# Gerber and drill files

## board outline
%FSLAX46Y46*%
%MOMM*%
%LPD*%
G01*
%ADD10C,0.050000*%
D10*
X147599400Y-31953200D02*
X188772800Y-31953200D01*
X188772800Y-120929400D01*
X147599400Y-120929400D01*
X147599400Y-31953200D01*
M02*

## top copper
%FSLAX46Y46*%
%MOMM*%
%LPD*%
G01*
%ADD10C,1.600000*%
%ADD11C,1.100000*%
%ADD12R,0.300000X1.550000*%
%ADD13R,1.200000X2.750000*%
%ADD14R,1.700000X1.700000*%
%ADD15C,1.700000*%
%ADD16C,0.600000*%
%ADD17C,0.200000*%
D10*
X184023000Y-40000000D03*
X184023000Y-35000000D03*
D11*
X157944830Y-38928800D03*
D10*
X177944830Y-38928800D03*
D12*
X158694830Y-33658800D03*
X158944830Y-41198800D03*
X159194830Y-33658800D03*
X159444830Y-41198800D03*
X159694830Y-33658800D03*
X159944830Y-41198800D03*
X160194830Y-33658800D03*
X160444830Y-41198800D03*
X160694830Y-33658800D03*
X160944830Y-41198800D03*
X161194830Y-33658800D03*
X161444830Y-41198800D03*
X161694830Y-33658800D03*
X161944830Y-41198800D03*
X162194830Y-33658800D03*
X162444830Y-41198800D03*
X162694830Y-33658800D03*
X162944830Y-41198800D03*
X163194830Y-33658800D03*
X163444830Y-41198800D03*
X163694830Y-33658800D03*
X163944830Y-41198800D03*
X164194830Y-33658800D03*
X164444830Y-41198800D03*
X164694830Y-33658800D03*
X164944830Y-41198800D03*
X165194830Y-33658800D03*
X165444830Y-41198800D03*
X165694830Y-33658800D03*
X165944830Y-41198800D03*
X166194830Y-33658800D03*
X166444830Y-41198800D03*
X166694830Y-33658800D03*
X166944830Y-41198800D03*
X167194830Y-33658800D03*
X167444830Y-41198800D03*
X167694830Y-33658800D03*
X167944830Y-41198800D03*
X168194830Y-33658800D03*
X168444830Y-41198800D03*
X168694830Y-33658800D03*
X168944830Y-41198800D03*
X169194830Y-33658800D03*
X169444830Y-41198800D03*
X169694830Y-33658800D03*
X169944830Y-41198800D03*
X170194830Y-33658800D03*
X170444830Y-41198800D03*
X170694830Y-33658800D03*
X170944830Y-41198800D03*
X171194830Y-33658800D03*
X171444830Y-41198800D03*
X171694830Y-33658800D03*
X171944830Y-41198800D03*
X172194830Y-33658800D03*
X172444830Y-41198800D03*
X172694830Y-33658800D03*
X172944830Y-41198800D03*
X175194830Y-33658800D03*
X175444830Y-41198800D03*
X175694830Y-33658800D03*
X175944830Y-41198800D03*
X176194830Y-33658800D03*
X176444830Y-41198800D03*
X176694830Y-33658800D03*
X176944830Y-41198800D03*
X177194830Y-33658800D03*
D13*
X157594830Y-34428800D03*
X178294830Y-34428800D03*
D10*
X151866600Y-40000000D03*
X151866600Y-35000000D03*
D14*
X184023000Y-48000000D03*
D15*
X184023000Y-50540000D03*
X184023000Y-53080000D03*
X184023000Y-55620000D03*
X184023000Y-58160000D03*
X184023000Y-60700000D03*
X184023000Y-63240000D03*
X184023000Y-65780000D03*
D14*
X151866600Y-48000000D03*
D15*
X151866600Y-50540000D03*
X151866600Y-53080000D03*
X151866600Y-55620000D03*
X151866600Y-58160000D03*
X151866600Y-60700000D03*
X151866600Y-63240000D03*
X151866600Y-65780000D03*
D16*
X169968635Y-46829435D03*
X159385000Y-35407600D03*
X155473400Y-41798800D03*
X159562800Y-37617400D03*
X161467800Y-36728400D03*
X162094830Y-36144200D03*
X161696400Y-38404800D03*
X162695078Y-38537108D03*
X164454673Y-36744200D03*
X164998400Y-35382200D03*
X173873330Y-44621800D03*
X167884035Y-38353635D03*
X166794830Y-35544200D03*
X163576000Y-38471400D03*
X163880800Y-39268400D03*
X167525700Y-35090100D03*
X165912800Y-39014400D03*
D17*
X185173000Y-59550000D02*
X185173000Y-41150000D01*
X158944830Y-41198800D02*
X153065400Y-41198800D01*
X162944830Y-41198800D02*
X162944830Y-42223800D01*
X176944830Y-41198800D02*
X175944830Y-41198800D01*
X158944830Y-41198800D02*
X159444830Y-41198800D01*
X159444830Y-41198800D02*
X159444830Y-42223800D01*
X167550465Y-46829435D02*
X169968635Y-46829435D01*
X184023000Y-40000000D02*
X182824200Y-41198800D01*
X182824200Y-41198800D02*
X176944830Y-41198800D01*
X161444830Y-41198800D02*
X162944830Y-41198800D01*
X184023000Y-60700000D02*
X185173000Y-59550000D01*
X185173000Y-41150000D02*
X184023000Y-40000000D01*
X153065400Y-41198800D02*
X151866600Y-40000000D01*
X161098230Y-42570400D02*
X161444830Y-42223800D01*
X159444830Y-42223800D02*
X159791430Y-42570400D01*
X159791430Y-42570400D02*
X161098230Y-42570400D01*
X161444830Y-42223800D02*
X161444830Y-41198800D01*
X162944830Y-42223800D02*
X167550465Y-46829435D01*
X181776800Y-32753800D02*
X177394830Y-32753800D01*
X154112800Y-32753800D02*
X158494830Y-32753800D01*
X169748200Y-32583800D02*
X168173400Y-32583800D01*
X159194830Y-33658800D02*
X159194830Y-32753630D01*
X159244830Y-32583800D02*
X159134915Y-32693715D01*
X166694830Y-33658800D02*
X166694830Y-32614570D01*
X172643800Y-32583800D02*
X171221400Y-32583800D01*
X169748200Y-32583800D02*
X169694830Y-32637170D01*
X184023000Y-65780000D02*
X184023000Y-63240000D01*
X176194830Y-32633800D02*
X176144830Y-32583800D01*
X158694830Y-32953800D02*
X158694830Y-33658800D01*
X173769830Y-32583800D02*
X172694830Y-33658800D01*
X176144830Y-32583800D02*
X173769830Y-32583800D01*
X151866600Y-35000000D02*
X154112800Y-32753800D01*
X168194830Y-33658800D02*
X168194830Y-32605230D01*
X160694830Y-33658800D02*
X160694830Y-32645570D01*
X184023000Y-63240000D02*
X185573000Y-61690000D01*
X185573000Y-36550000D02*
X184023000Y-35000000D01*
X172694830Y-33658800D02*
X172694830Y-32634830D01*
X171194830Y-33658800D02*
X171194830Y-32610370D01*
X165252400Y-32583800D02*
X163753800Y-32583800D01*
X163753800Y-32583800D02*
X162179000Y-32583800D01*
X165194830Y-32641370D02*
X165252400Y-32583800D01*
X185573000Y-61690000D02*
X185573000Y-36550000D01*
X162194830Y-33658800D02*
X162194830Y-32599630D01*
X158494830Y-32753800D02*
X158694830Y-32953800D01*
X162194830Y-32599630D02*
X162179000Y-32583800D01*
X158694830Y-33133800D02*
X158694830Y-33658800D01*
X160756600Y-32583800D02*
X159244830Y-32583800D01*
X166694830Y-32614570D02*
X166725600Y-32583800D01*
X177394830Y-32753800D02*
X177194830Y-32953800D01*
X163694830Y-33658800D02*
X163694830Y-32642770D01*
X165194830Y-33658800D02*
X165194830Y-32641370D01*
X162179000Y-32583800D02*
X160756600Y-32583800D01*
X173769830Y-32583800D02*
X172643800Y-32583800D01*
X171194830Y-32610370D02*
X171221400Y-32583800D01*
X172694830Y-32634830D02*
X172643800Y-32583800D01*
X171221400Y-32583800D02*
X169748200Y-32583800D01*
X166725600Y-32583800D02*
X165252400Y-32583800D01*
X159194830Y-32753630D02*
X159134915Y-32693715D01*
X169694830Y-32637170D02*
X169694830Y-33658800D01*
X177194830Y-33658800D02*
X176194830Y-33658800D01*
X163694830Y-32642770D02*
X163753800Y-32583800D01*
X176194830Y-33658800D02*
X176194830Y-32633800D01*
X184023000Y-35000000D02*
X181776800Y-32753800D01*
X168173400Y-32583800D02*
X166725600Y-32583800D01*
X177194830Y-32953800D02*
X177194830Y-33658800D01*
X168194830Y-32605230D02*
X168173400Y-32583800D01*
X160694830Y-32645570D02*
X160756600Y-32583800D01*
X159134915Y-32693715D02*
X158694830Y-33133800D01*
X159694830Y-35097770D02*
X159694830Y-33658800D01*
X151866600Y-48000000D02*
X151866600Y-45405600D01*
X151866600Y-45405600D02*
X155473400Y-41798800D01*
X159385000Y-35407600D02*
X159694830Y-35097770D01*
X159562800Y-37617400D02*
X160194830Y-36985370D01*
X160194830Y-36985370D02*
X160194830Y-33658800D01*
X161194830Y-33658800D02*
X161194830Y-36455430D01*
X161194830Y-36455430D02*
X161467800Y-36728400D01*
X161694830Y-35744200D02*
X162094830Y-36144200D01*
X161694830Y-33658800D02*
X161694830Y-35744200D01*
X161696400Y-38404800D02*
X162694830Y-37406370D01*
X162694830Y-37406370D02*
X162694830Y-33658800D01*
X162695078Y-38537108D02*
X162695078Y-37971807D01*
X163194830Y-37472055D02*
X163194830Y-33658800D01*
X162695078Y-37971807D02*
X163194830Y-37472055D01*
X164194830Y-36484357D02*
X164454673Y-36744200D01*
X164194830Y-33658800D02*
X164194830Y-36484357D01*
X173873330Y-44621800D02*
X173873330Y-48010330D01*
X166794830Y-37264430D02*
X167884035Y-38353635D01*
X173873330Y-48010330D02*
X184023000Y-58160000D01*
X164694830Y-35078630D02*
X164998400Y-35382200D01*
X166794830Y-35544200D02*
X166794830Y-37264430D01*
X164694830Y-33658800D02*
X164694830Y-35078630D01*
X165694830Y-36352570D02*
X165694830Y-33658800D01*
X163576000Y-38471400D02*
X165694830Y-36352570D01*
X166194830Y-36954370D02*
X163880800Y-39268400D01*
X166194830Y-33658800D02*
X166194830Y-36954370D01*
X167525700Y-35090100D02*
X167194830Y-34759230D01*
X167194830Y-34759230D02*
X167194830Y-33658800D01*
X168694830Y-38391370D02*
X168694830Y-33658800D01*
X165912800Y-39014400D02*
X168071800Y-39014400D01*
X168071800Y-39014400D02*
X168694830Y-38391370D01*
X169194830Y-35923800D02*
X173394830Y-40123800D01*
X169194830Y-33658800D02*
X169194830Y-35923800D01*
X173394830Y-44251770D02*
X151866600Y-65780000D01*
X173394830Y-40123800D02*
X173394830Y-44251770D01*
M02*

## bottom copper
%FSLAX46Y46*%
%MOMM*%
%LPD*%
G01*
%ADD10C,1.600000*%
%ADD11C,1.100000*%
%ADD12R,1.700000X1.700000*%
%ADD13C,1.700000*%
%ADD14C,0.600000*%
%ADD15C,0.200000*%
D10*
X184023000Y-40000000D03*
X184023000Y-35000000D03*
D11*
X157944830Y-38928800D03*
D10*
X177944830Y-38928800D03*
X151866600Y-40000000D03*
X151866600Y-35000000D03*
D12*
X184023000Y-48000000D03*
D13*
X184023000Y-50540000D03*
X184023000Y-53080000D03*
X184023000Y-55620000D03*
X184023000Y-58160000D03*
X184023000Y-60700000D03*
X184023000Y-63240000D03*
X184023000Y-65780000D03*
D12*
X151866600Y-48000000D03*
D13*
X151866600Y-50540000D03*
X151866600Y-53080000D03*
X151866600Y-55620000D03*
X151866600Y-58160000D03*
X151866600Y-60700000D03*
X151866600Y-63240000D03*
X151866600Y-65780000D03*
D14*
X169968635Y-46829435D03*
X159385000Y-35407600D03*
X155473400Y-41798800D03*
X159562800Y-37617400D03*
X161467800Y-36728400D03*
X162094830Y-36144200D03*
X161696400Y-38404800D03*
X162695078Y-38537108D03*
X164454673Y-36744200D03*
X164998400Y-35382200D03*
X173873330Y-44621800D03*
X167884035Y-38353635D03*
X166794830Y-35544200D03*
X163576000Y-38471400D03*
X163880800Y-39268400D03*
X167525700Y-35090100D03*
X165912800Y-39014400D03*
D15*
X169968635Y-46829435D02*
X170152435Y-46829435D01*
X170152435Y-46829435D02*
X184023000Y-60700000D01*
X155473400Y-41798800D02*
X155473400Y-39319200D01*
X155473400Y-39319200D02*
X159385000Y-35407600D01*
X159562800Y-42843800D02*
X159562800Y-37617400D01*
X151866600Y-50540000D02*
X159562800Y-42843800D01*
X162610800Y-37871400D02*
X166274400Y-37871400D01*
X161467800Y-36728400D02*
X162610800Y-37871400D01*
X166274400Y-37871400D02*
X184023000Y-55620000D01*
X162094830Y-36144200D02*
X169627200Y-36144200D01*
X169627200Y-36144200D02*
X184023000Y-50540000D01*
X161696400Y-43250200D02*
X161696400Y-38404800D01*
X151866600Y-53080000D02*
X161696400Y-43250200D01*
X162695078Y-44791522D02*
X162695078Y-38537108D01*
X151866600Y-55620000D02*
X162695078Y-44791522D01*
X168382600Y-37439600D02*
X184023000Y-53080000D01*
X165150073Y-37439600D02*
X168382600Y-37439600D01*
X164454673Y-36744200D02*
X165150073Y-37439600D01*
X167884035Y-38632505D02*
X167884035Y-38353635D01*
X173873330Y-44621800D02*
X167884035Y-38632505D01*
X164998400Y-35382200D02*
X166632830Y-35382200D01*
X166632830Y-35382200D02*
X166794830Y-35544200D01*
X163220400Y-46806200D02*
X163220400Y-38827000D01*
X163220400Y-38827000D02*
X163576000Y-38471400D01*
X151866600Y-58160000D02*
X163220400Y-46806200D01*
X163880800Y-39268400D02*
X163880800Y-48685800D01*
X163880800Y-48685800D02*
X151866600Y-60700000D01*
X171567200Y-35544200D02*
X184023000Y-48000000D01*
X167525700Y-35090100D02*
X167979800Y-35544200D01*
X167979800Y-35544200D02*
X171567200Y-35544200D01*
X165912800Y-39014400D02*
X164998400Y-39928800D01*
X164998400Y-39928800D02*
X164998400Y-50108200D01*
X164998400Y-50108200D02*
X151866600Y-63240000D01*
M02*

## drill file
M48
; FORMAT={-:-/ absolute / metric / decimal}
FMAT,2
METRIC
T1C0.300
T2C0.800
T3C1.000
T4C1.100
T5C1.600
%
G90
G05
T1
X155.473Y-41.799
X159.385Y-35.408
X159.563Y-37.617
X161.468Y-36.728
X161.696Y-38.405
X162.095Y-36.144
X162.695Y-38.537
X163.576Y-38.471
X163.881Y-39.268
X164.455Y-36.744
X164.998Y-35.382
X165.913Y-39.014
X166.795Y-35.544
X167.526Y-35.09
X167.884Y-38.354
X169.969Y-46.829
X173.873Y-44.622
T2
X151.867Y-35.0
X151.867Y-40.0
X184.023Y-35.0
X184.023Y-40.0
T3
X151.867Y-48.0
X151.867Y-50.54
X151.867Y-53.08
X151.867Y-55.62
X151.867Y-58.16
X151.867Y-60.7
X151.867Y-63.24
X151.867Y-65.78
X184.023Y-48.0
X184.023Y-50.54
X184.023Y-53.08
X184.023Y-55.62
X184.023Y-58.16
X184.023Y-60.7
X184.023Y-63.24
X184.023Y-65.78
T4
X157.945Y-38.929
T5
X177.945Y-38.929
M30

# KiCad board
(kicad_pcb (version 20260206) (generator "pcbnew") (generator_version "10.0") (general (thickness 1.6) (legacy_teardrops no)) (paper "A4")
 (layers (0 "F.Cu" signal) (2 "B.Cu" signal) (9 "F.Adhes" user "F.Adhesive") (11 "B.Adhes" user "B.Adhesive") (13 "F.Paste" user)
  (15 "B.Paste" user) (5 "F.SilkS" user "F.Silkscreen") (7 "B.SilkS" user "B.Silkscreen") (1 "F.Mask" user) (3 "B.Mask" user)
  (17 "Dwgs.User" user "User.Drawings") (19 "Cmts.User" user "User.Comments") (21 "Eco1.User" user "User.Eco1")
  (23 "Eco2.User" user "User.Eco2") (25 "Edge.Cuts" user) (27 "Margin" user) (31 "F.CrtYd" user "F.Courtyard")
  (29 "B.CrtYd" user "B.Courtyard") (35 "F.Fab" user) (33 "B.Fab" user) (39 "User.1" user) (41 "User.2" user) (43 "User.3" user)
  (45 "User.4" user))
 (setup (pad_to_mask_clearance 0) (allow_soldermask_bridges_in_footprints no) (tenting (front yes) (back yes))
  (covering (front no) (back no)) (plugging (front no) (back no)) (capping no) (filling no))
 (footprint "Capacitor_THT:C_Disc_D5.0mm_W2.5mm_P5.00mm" (layer "F.Cu") (at 184.023 40 90)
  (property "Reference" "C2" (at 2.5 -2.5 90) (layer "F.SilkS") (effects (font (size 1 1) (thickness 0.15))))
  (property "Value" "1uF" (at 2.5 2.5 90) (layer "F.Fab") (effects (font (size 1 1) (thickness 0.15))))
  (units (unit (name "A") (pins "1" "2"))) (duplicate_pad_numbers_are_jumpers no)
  (pad "1" thru_hole circle (at 0 0 90) (size 1.6 1.6) (drill 0.8) (layers "*.Cu" "*.Mask") (remove_unused_layers no) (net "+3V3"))
  (pad "2" thru_hole circle (at 5 0 90) (size 1.6 1.6) (drill 0.8) (layers "*.Cu" "*.Mask") (remove_unused_layers no) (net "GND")))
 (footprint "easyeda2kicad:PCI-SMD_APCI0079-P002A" (layer "F.Cu") (at 167.94483 37.4288)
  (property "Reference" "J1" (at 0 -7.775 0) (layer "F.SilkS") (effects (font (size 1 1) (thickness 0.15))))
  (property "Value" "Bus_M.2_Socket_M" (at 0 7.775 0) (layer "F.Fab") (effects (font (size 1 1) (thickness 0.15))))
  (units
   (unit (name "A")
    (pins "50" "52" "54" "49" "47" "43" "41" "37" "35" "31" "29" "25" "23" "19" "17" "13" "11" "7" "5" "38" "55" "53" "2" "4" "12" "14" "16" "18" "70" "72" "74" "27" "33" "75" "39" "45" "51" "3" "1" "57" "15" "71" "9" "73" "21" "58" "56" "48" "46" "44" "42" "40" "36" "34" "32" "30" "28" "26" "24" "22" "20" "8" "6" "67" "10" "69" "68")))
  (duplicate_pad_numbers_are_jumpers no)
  (pad "" thru_hole circle (at -10 1.5) (size 1.1 1.1) (drill 1.1) (layers "*.Cu" "*.Mask") (remove_unused_layers no))
  (pad "" thru_hole circle (at 10 1.5) (size 1.6 1.6) (drill 1.6) (layers "*.Cu" "*.Mask") (remove_unused_layers no))
  (pad "1" smd rect (at -9.25 -3.77) (size 0.3 1.55) (layers "F.Cu" "F.Mask" "F.Paste") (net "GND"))
  (pad "2" smd rect (at -9 3.77) (size 0.3 1.55) (layers "F.Cu" "F.Mask" "F.Paste") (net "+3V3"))
  (pad "3" smd rect (at -8.75 -3.77) (size 0.3 1.55) (layers "F.Cu" "F.Mask" "F.Paste") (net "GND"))
  (pad "4" smd rect (at -8.5 3.77) (size 0.3 1.55) (layers "F.Cu" "F.Mask" "F.Paste") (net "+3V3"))
  (pad "5" smd rect (at -8.25 -3.77) (size 0.3 1.55) (layers "F.Cu" "F.Mask" "F.Paste") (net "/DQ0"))
  (pad "6" smd rect (at -8 3.77) (size 0.3 1.55) (layers "F.Cu" "F.Mask" "F.Paste") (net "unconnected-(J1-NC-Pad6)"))
  (pad "7" smd rect (at -7.75 -3.77) (size 0.3 1.55) (layers "F.Cu" "F.Mask" "F.Paste") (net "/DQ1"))
  (pad "8" smd rect (at -7.5 3.77) (size 0.3 1.55) (layers "F.Cu" "F.Mask" "F.Paste") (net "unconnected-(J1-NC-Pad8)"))
  (pad "9" smd rect (at -7.25 -3.77) (size 0.3 1.55) (layers "F.Cu" "F.Mask" "F.Paste") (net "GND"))
  (pad "10" smd rect (at -7 3.77) (size 0.3 1.55) (layers "F.Cu" "F.Mask" "F.Paste")
   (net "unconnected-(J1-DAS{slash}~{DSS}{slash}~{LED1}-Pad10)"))
  (pad "11" smd rect (at -6.75 -3.77) (size 0.3 1.55) (layers "F.Cu" "F.Mask" "F.Paste") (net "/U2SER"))
  (pad "12" smd rect (at -6.5 3.77) (size 0.3 1.55) (layers "F.Cu" "F.Mask" "F.Paste") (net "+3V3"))
  (pad "13" smd rect (at -6.25 -3.77) (size 0.3 1.55) (layers "F.Cu" "F.Mask" "F.Paste") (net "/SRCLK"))
  (pad "14" smd rect (at -6 3.77) (size 0.3 1.55) (layers "F.Cu" "F.Mask" "F.Paste") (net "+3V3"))
  (pad "15" smd rect (at -5.75 -3.77) (size 0.3 1.55) (layers "F.Cu" "F.Mask" "F.Paste") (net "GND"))
  (pad "16" smd rect (at -5.5 3.77) (size 0.3 1.55) (layers "F.Cu" "F.Mask" "F.Paste") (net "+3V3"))
  (pad "17" smd rect (at -5.25 -3.77) (size 0.3 1.55) (layers "F.Cu" "F.Mask" "F.Paste") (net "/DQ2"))
  (pad "18" smd rect (at -5 3.77) (size 0.3 1.55) (layers "F.Cu" "F.Mask" "F.Paste") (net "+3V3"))
  (pad "19" smd rect (at -4.75 -3.77) (size 0.3 1.55) (layers "F.Cu" "F.Mask" "F.Paste") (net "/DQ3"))
  (pad "20" smd rect (at -4.5 3.77) (size 0.3 1.55) (layers "F.Cu" "F.Mask" "F.Paste") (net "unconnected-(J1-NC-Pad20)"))
  (pad "21" smd rect (at -4.25 -3.77) (size 0.3 1.55) (layers "F.Cu" "F.Mask" "F.Paste") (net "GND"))
  (pad "22" smd rect (at -4 3.77) (size 0.3 1.55) (layers "F.Cu" "F.Mask" "F.Paste") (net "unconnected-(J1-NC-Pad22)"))
  (pad "23" smd rect (at -3.75 -3.77) (size 0.3 1.55) (layers "F.Cu" "F.Mask" "F.Paste") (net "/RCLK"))
  (pad "24" smd rect (at -3.5 3.77) (size 0.3 1.55) (layers "F.Cu" "F.Mask" "F.Paste") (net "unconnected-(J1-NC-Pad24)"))
  (pad "25" smd rect (at -3.25 -3.77) (size 0.3 1.55) (layers "F.Cu" "F.Mask" "F.Paste") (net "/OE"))
  (pad "26" smd rect (at -3 3.77) (size 0.3 1.55) (layers "F.Cu" "F.Mask" "F.Paste") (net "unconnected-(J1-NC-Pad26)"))
  (pad "27" smd rect (at -2.75 -3.77) (size 0.3 1.55) (layers "F.Cu" "F.Mask" "F.Paste") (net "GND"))
  (pad "28" smd rect (at -2.5 3.77) (size 0.3 1.55) (layers "F.Cu" "F.Mask" "F.Paste") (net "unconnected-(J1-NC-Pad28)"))
  (pad "29" smd rect (at -2.25 -3.77) (size 0.3 1.55) (layers "F.Cu" "F.Mask" "F.Paste") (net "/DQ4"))
  (pad "30" smd rect (at -2 3.77) (size 0.3 1.55) (layers "F.Cu" "F.Mask" "F.Paste") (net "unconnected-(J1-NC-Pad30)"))
  (pad "31" smd rect (at -1.75 -3.77) (size 0.3 1.55) (layers "F.Cu" "F.Mask" "F.Paste") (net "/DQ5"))
  (pad "32" smd rect (at -1.5 3.77) (size 0.3 1.55) (layers "F.Cu" "F.Mask" "F.Paste") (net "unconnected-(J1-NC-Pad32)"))
  (pad "33" smd rect (at -1.25 -3.77) (size 0.3 1.55) (layers "F.Cu" "F.Mask" "F.Paste") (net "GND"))
  (pad "34" smd rect (at -1 3.77) (size 0.3 1.55) (layers "F.Cu" "F.Mask" "F.Paste") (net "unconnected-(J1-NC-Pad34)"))
  (pad "35" smd rect (at -0.75 -3.77) (size 0.3 1.55) (layers "F.Cu" "F.Mask" "F.Paste") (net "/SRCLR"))
  (pad "36" smd rect (at -0.5 3.77) (size 0.3 1.55) (layers "F.Cu" "F.Mask" "F.Paste") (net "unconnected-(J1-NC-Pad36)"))
  (pad "37" smd rect (at -0.25 -3.77) (size 0.3 1.55) (layers "F.Cu" "F.Mask" "F.Paste") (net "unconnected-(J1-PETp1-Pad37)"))
  (pad "38" smd rect (at 0 3.77) (size 0.3 1.55) (layers "F.Cu" "F.Mask" "F.Paste") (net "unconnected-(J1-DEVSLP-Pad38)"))
  (pad "39" smd rect (at 0.25 -3.77) (size 0.3 1.55) (layers "F.Cu" "F.Mask" "F.Paste") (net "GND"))
  (pad "40" smd rect (at 0.5 3.77) (size 0.3 1.55) (layers "F.Cu" "F.Mask" "F.Paste") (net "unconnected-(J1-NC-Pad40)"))
  (pad "41" smd rect (at 0.75 -3.77) (size 0.3 1.55) (layers "F.Cu" "F.Mask" "F.Paste") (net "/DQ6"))
  (pad "42" smd rect (at 1 3.77) (size 0.3 1.55) (layers "F.Cu" "F.Mask" "F.Paste") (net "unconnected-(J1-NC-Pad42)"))
  (pad "43" smd rect (at 1.25 -3.77) (size 0.3 1.55) (layers "F.Cu" "F.Mask" "F.Paste") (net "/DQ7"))
  (pad "44" smd rect (at 1.5 3.77) (size 0.3 1.55) (layers "F.Cu" "F.Mask" "F.Paste") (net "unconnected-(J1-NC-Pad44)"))
  (pad "45" smd rect (at 1.75 -3.77) (size 0.3 1.55) (layers "F.Cu" "F.Mask" "F.Paste") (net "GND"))
  (pad "46" smd rect (at 2 3.77) (size 0.3 1.55) (layers "F.Cu" "F.Mask" "F.Paste") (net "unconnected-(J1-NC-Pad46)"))
  (pad "47" smd rect (at 2.25 -3.77) (size 0.3 1.55) (layers "F.Cu" "F.Mask" "F.Paste") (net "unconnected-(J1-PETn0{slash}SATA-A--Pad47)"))
  (pad "48" smd rect (at 2.5 3.77) (size 0.3 1.55) (layers "F.Cu" "F.Mask" "F.Paste") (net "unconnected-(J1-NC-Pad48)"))
  (pad "49" smd rect (at 2.75 -3.77) (size 0.3 1.55) (layers "F.Cu" "F.Mask" "F.Paste") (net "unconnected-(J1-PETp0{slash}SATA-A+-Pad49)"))
  (pad "50" smd rect (at 3 3.77) (size 0.3 1.55) (layers "F.Cu" "F.Mask" "F.Paste") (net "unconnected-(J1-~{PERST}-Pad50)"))
  (pad "51" smd rect (at 3.25 -3.77) (size 0.3 1.55) (layers "F.Cu" "F.Mask" "F.Paste") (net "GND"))
  (pad "52" smd rect (at 3.5 3.77) (size 0.3 1.55) (layers "F.Cu" "F.Mask" "F.Paste") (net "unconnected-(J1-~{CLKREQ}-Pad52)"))
  (pad "53" smd rect (at 3.75 -3.77) (size 0.3 1.55) (layers "F.Cu" "F.Mask" "F.Paste") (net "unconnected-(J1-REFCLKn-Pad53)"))
  (pad "54" smd rect (at 4 3.77) (size 0.3 1.55) (layers "F.Cu" "F.Mask" "F.Paste") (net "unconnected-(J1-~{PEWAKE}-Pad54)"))
  (pad "55" smd rect (at 4.25 -3.77) (size 0.3 1.55) (layers "F.Cu" "F.Mask" "F.Paste") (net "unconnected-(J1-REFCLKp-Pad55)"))
  (pad "56" smd rect (at 4.5 3.77) (size 0.3 1.55) (layers "F.Cu" "F.Mask" "F.Paste") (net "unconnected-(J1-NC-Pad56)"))
  (pad "57" smd rect (at 4.75 -3.77) (size 0.3 1.55) (layers "F.Cu" "F.Mask" "F.Paste") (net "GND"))
  (pad "58" smd rect (at 5 3.77) (size 0.3 1.55) (layers "F.Cu" "F.Mask" "F.Paste") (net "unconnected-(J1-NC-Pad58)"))
  (pad "67" smd rect (at 7.25 -3.77) (size 0.3 1.55) (layers "F.Cu" "F.Mask" "F.Paste") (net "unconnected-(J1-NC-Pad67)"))
  (pad "68" smd rect (at 7.5 3.77) (size 0.3 1.55) (layers "F.Cu" "F.Mask" "F.Paste") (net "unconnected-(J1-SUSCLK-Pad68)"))
  (pad "69" smd rect (at 7.75 -3.77) (size 0.3 1.55) (layers "F.Cu" "F.Mask" "F.Paste") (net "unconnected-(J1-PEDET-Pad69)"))
  (pad "70" smd rect (at 8 3.77) (size 0.3 1.55) (layers "F.Cu" "F.Mask" "F.Paste") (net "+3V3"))
  (pad "71" smd rect (at 8.25 -3.77) (size 0.3 1.55) (layers "F.Cu" "F.Mask" "F.Paste") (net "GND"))
  (pad "72" smd rect (at 8.5 3.77) (size 0.3 1.55) (layers "F.Cu" "F.Mask" "F.Paste") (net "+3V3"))
  (pad "73" smd rect (at 8.75 -3.77) (size 0.3 1.55) (layers "F.Cu" "F.Mask" "F.Paste") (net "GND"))
  (pad "74" smd rect (at 9 3.77) (size 0.3 1.55) (layers "F.Cu" "F.Mask" "F.Paste") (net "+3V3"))
  (pad "75" smd rect (at 9.25 -3.77) (size 0.3 1.55) (layers "F.Cu" "F.Mask" "F.Paste") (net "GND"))
  (pad "76" smd rect (at -10.35 -3) (size 1.2 2.75) (layers "F.Cu" "F.Mask" "F.Paste"))
  (pad "76" smd rect (at 10.35 -3) (size 1.2 2.75) (layers "F.Cu" "F.Mask" "F.Paste")))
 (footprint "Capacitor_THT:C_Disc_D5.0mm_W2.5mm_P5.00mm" (layer "F.Cu") (at 151.8666 40 90)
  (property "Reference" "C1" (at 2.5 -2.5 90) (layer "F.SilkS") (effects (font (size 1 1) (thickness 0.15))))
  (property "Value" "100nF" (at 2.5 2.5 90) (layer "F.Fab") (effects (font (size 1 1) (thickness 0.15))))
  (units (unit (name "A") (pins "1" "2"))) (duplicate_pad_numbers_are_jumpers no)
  (pad "1" thru_hole circle (at 0 0 90) (size 1.6 1.6) (drill 0.8) (layers "*.Cu" "*.Mask") (remove_unused_layers no) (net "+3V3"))
  (pad "2" thru_hole circle (at 5 0 90) (size 1.6 1.6) (drill 0.8) (layers "*.Cu" "*.Mask") (remove_unused_layers no) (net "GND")))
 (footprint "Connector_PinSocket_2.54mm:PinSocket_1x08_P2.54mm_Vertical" (layer "F.Cu") (at 184.023 48)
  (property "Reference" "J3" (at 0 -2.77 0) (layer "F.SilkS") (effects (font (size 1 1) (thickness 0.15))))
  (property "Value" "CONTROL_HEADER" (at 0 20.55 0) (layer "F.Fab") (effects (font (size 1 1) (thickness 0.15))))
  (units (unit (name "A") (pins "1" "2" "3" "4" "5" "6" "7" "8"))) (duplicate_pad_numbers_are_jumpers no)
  (pad "1" thru_hole rect (at 0 0) (size 1.7 1.7) (drill 1) (layers "*.Cu" "*.Mask") (remove_unused_layers no) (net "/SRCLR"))
  (pad "2" thru_hole circle (at 0 2.54) (size 1.7 1.7) (drill 1) (layers "*.Cu" "*.Mask") (remove_unused_layers no) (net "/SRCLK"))
  (pad "3" thru_hole circle (at 0 5.08) (size 1.7 1.7) (drill 1) (layers "*.Cu" "*.Mask") (remove_unused_layers no) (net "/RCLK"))
  (pad "4" thru_hole circle (at 0 7.62) (size 1.7 1.7) (drill 1) (layers "*.Cu" "*.Mask") (remove_unused_layers no) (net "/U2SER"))
  (pad "5" thru_hole circle (at 0 10.16) (size 1.7 1.7) (drill 1) (layers "*.Cu" "*.Mask") (remove_unused_layers no) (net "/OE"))
  (pad "6" thru_hole circle (at 0 12.7) (size 1.7 1.7) (drill 1) (layers "*.Cu" "*.Mask") (remove_unused_layers no) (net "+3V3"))
  (pad "7" thru_hole circle (at 0 15.24) (size 1.7 1.7) (drill 1) (layers "*.Cu" "*.Mask") (remove_unused_layers no) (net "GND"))
  (pad "8" thru_hole circle (at 0 17.78) (size 1.7 1.7) (drill 1) (layers "*.Cu" "*.Mask") (remove_unused_layers no) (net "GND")))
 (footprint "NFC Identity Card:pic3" (layer "F.Cu") (at 168.148 111.0488)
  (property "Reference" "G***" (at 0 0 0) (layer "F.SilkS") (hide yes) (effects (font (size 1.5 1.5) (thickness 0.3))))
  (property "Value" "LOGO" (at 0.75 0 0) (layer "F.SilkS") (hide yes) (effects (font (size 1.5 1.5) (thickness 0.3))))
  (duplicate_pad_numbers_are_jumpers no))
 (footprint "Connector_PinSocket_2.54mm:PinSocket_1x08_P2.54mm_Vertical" (layer "F.Cu") (at 151.8666 48)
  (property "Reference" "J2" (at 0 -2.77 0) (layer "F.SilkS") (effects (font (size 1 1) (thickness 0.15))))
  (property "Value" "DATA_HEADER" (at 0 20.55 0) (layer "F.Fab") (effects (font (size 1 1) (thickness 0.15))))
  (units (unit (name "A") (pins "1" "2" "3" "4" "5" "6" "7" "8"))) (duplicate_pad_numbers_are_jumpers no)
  (pad "1" thru_hole rect (at 0 0) (size 1.7 1.7) (drill 1) (layers "*.Cu" "*.Mask") (remove_unused_layers no) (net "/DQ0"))
  (pad "2" thru_hole circle (at 0 2.54) (size 1.7 1.7) (drill 1) (layers "*.Cu" "*.Mask") (remove_unused_layers no) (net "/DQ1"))
  (pad "3" thru_hole circle (at 0 5.08) (size 1.7 1.7) (drill 1) (layers "*.Cu" "*.Mask") (remove_unused_layers no) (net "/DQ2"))
  (pad "4" thru_hole circle (at 0 7.62) (size 1.7 1.7) (drill 1) (layers "*.Cu" "*.Mask") (remove_unused_layers no) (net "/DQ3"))
  (pad "5" thru_hole circle (at 0 10.16) (size 1.7 1.7) (drill 1) (layers "*.Cu" "*.Mask") (remove_unused_layers no) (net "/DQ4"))
  (pad "6" thru_hole circle (at 0 12.7) (size 1.7 1.7) (drill 1) (layers "*.Cu" "*.Mask") (remove_unused_layers no) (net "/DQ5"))
  (pad "7" thru_hole circle (at 0 15.24) (size 1.7 1.7) (drill 1) (layers "*.Cu" "*.Mask") (remove_unused_layers no) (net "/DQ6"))
  (pad "8" thru_hole circle (at 0 17.78) (size 1.7 1.7) (drill 1) (layers "*.Cu" "*.Mask") (remove_unused_layers no) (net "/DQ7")))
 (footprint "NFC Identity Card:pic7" (layer "B.Cu") (at 168.8592 117.348 180)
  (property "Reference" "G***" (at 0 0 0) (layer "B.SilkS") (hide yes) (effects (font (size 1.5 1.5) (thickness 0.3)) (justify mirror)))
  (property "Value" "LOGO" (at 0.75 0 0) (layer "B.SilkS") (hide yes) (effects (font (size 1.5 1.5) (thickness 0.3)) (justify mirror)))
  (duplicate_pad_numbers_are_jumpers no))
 (gr_rect (start 147.5994 31.9532) (end 188.7728 120.9294) (stroke (width 0.05) (type default)) (fill no) (layer "Edge.Cuts"))
 (segment (start 185.173 59.55) (end 185.173 41.15) (width 0.2) (layer "F.Cu") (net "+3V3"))
 (segment (start 158.94483 41.1988) (end 153.0654 41.1988) (width 0.2) (layer "F.Cu") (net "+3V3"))
 (segment (start 162.94483 41.1988) (end 162.94483 42.2238) (width 0.2) (layer "F.Cu") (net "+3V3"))
 (segment (start 176.94483 41.1988) (end 175.94483 41.1988) (width 0.2) (layer "F.Cu") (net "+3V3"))
 (segment (start 158.94483 41.1988) (end 159.44483 41.1988) (width 0.2) (layer "F.Cu") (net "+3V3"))
 (segment (start 159.44483 41.1988) (end 159.44483 42.2238) (width 0.2) (layer "F.Cu") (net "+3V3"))
 (segment (start 167.550465 46.829435) (end 169.968635 46.829435) (width 0.2) (layer "F.Cu") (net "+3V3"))
 (segment (start 184.023 40) (end 182.8242 41.1988) (width 0.2) (layer "F.Cu") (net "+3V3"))
 (segment (start 182.8242 41.1988) (end 176.94483 41.1988) (width 0.2) (layer "F.Cu") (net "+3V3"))
 (segment (start 161.44483 41.1988) (end 162.94483 41.1988) (width 0.2) (layer "F.Cu") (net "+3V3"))
 (segment (start 184.023 60.7) (end 185.173 59.55) (width 0.2) (layer "F.Cu") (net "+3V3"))
 (segment (start 185.173 41.15) (end 184.023 40) (width 0.2) (layer "F.Cu") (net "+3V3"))
 (segment (start 153.0654 41.1988) (end 151.8666 40) (width 0.2) (layer "F.Cu") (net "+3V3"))
 (segment (start 161.09823 42.5704) (end 161.44483 42.2238) (width 0.2) (layer "F.Cu") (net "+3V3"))
 (segment (start 159.44483 42.2238) (end 159.79143 42.5704) (width 0.2) (layer "F.Cu") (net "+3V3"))
 (segment (start 159.79143 42.5704) (end 161.09823 42.5704) (width 0.2) (layer "F.Cu") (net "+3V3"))
 (segment (start 161.44483 42.2238) (end 161.44483 41.1988) (width 0.2) (layer "F.Cu") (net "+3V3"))
 (segment (start 162.94483 42.2238) (end 167.550465 46.829435) (width 0.2) (layer "F.Cu") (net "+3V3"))
 (via (at 169.968635 46.829435) (size 0.6) (drill 0.3) (layers "F.Cu" "B.Cu") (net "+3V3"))
 (segment (start 169.968635 46.829435) (end 170.152435 46.829435) (width 0.2) (layer "B.Cu") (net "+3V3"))
 (segment (start 170.152435 46.829435) (end 184.023 60.7) (width 0.2) (layer "B.Cu") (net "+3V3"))
 (segment (start 181.7768 32.7538) (end 177.39483 32.7538) (width 0.2) (layer "F.Cu") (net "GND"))
 (segment (start 154.1128 32.7538) (end 158.49483 32.7538) (width 0.2) (layer "F.Cu") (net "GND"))
 (segment (start 169.7482 32.5838) (end 168.1734 32.5838) (width 0.2) (layer "F.Cu") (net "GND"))
 (segment (start 159.19483 33.6588) (end 159.19483 32.75363) (width 0.2) (layer "F.Cu") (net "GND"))
 (segment (start 159.24483 32.5838) (end 159.134915 32.693715) (width 0.2) (layer "F.Cu") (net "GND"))
 (segment (start 166.69483 33.6588) (end 166.69483 32.61457) (width 0.2) (layer "F.Cu") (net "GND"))
 (segment (start 172.6438 32.5838) (end 171.2214 32.5838) (width 0.2) (layer "F.Cu") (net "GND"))
 (segment (start 169.7482 32.5838) (end 169.69483 32.63717) (width 0.2) (layer "F.Cu") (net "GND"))
 (segment (start 184.023 65.78) (end 184.023 63.24) (width 0.2) (layer "F.Cu") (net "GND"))
 (segment (start 176.19483 32.6338) (end 176.14483 32.5838) (width 0.2) (layer "F.Cu") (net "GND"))
 (segment (start 158.69483 32.9538) (end 158.69483 33.6588) (width 0.2) (layer "F.Cu") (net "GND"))
 (segment (start 173.76983 32.5838) (end 172.69483 33.6588) (width 0.2) (layer "F.Cu") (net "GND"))
 (segment (start 176.14483 32.5838) (end 173.76983 32.5838) (width 0.2) (layer "F.Cu") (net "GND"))
 (segment (start 151.8666 35) (end 154.1128 32.7538) (width 0.2) (layer "F.Cu") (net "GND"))
 (segment (start 168.19483 33.6588) (end 168.19483 32.60523) (width 0.2) (layer "F.Cu") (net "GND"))
 (segment (start 160.69483 33.6588) (end 160.69483 32.64557) (width 0.2) (layer "F.Cu") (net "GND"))
 (segment (start 184.023 63.24) (end 185.573 61.69) (width 0.2) (layer "F.Cu") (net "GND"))
 (segment (start 185.573 36.55) (end 184.023 35) (width 0.2) (layer "F.Cu") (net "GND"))
 (segment (start 172.69483 33.6588) (end 172.69483 32.63483) (width 0.2) (layer "F.Cu") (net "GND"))
 (segment (start 171.19483 33.6588) (end 171.19483 32.61037) (width 0.2) (layer "F.Cu") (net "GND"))
 (segment (start 165.2524 32.5838) (end 163.7538 32.5838) (width 0.2) (layer "F.Cu") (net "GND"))
 (segment (start 163.7538 32.5838) (end 162.179 32.5838) (width 0.2) (layer "F.Cu") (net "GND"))
 (segment (start 165.19483 32.64137) (end 165.2524 32.5838) (width 0.2) (layer "F.Cu") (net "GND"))
 (segment (start 185.573 61.69) (end 185.573 36.55) (width 0.2) (layer "F.Cu") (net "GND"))
 (segment (start 162.19483 33.6588) (end 162.19483 32.59963) (width 0.2) (layer "F.Cu") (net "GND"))
 (segment (start 158.49483 32.7538) (end 158.69483 32.9538) (width 0.2) (layer "F.Cu") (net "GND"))
 (segment (start 162.19483 32.59963) (end 162.179 32.5838) (width 0.2) (layer "F.Cu") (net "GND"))
 (segment (start 158.69483 33.1338) (end 158.69483 33.6588) (width 0.2) (layer "F.Cu") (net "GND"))
 (segment (start 160.7566 32.5838) (end 159.24483 32.5838) (width 0.2) (layer "F.Cu") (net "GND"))
 (segment (start 166.69483 32.61457) (end 166.7256 32.5838) (width 0.2) (layer "F.Cu") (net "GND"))
 (segment (start 177.39483 32.7538) (end 177.19483 32.9538) (width 0.2) (layer "F.Cu") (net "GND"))
 (segment (start 163.69483 33.6588) (end 163.69483 32.64277) (width 0.2) (layer "F.Cu") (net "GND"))
 (segment (start 165.19483 33.6588) (end 165.19483 32.64137) (width 0.2) (layer "F.Cu") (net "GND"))
 (segment (start 162.179 32.5838) (end 160.7566 32.5838) (width 0.2) (layer "F.Cu") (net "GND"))
 (segment (start 173.76983 32.5838) (end 172.6438 32.5838) (width 0.2) (layer "F.Cu") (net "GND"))
 (segment (start 171.19483 32.61037) (end 171.2214 32.5838) (width 0.2) (layer "F.Cu") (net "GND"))
 (segment (start 172.69483 32.63483) (end 172.6438 32.5838) (width 0.2) (layer "F.Cu") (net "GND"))
 (segment (start 171.2214 32.5838) (end 169.7482 32.5838) (width 0.2) (layer "F.Cu") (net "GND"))
 (segment (start 166.7256 32.5838) (end 165.2524 32.5838) (width 0.2) (layer "F.Cu") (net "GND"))
 (segment (start 159.19483 32.75363) (end 159.134915 32.693715) (width 0.2) (layer "F.Cu") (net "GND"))
 (segment (start 169.69483 32.63717) (end 169.69483 33.6588) (width 0.2) (layer "F.Cu") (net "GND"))
 (segment (start 177.19483 33.6588) (end 176.19483 33.6588) (width 0.2) (layer "F.Cu") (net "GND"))
 (segment (start 163.69483 32.64277) (end 163.7538 32.5838) (width 0.2) (layer "F.Cu") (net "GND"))
 (segment (start 176.19483 33.6588) (end 176.19483 32.6338) (width 0.2) (layer "F.Cu") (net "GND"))
 (segment (start 184.023 35) (end 181.7768 32.7538) (width 0.2) (layer "F.Cu") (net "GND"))
 (segment (start 168.1734 32.5838) (end 166.7256 32.5838) (width 0.2) (layer "F.Cu") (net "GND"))
 (segment (start 177.19483 32.9538) (end 177.19483 33.6588) (width 0.2) (layer "F.Cu") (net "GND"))
 (segment (start 168.19483 32.60523) (end 168.1734 32.5838) (width 0.2) (layer "F.Cu") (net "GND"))
 (segment (start 160.69483 32.64557) (end 160.7566 32.5838) (width 0.2) (layer "F.Cu") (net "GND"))
 (segment (start 159.134915 32.693715) (end 158.69483 33.1338) (width 0.2) (layer "F.Cu") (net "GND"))
 (segment (start 159.69483 35.09777) (end 159.69483 33.6588) (width 0.2) (layer "F.Cu") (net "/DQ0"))
 (segment (start 151.8666 48) (end 151.8666 45.4056) (width 0.2) (layer "F.Cu") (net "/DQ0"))
 (segment (start 151.8666 45.4056) (end 155.4734 41.7988) (width 0.2) (layer "F.Cu") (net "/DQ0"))
 (segment (start 159.385 35.4076) (end 159.69483 35.09777) (width 0.2) (layer "F.Cu") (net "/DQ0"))
 (via (at 159.385 35.4076) (size 0.6) (drill 0.3) (layers "F.Cu" "B.Cu") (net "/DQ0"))
 (via (at 155.4734 41.7988) (size 0.6) (drill 0.3) (layers "F.Cu" "B.Cu") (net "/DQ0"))
 (segment (start 155.4734 41.7988) (end 155.4734 39.3192) (width 0.2) (layer "B.Cu") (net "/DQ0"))
 (segment (start 155.4734 39.3192) (end 159.385 35.4076) (width 0.2) (layer "B.Cu") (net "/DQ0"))
 (segment (start 159.5628 37.6174) (end 160.19483 36.98537) (width 0.2) (layer "F.Cu") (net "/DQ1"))
 (segment (start 160.19483 36.98537) (end 160.19483 33.6588) (width 0.2) (layer "F.Cu") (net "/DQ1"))
 (via (at 159.5628 37.6174) (size 0.6) (drill 0.3) (layers "F.Cu" "B.Cu") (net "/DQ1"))
 (segment (start 159.5628 42.8438) (end 159.5628 37.6174) (width 0.2) (layer "B.Cu") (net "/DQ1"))
 (segment (start 151.8666 50.54) (end 159.5628 42.8438) (width 0.2) (layer "B.Cu") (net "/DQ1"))
 (segment (start 161.19483 33.6588) (end 161.19483 36.45543) (width 0.2) (layer "F.Cu") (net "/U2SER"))
 (segment (start 161.19483 36.45543) (end 161.4678 36.7284) (width 0.2) (layer "F.Cu") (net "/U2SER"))
 (via (at 161.4678 36.7284) (size 0.6) (drill 0.3) (layers "F.Cu" "B.Cu") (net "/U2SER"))
 (segment (start 162.6108 37.8714) (end 166.2744 37.8714) (width 0.2) (layer "B.Cu") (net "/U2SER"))
 (segment (start 161.4678 36.7284) (end 162.6108 37.8714) (width 0.2) (layer "B.Cu") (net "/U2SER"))
 (segment (start 166.2744 37.8714) (end 184.023 55.62) (width 0.2) (layer "B.Cu") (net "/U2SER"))
 (segment (start 161.69483 35.7442) (end 162.09483 36.1442) (width 0.2) (layer "F.Cu") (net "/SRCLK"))
 (segment (start 161.69483 33.6588) (end 161.69483 35.7442) (width 0.2) (layer "F.Cu") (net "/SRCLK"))
 (via (at 162.09483 36.1442) (size 0.6) (drill 0.3) (layers "F.Cu" "B.Cu") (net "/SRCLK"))
 (segment (start 162.09483 36.1442) (end 169.6272 36.1442) (width 0.2) (layer "B.Cu") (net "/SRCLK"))
 (segment (start 169.6272 36.1442) (end 184.023 50.54) (width 0.2) (layer "B.Cu") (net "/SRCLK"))
 (segment (start 161.6964 38.4048) (end 162.69483 37.40637) (width 0.2) (layer "F.Cu") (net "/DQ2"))
 (segment (start 162.69483 37.40637) (end 162.69483 33.6588) (width 0.2) (layer "F.Cu") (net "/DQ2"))
 (via (at 161.6964 38.4048) (size 0.6) (drill 0.3) (layers "F.Cu" "B.Cu") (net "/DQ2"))
 (segment (start 161.6964 43.2502) (end 161.6964 38.4048) (width 0.2) (layer "B.Cu") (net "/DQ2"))
 (segment (start 151.8666 53.08) (end 161.6964 43.2502) (width 0.2) (layer "B.Cu") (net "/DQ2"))
 (segment (start 162.695078 38.537108) (end 162.695078 37.971807) (width 0.2) (layer "F.Cu") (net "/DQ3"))
 (segment (start 163.19483 37.472055) (end 163.19483 33.6588) (width 0.2) (layer "F.Cu") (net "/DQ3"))
 (segment (start 162.695078 37.971807) (end 163.19483 37.472055) (width 0.2) (layer "F.Cu") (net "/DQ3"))
 (via (at 162.695078 38.537108) (size 0.6) (drill 0.3) (layers "F.Cu" "B.Cu") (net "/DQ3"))
 (segment (start 162.695078 44.791522) (end 162.695078 38.537108) (width 0.2) (layer "B.Cu") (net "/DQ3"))
 (segment (start 151.8666 55.62) (end 162.695078 44.791522) (width 0.2) (layer "B.Cu") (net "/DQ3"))
 (segment (start 164.19483 36.484357) (end 164.454673 36.7442) (width 0.2) (layer "F.Cu") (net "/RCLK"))
 (segment (start 164.19483 33.6588) (end 164.19483 36.484357) (width 0.2) (layer "F.Cu") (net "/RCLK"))
 (via (at 164.454673 36.7442) (size 0.6) (drill 0.3) (layers "F.Cu" "B.Cu") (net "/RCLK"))
 (segment (start 168.3826 37.4396) (end 184.023 53.08) (width 0.2) (layer "B.Cu") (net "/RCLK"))
 (segment (start 165.150073 37.4396) (end 168.3826 37.4396) (width 0.2) (layer "B.Cu") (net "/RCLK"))
 (segment (start 164.454673 36.7442) (end 165.150073 37.4396) (width 0.2) (layer "B.Cu") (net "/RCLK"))
 (segment (start 173.87333 44.6218) (end 173.87333 48.01033) (width 0.2) (layer "F.Cu") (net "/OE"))
 (segment (start 166.79483 37.26443) (end 167.884035 38.353635) (width 0.2) (layer "F.Cu") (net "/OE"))
 (segment (start 173.87333 48.01033) (end 184.023 58.16) (width 0.2) (layer "F.Cu") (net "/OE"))
 (segment (start 164.69483 35.07863) (end 164.9984 35.3822) (width 0.2) (layer "F.Cu") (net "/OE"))
 (segment (start 166.79483 35.5442) (end 166.79483 37.26443) (width 0.2) (layer "F.Cu") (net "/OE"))
 (segment (start 164.69483 33.6588) (end 164.69483 35.07863) (width 0.2) (layer "F.Cu") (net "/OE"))
 (via (at 164.9984 35.3822) (size 0.6) (drill 0.3) (layers "F.Cu" "B.Cu") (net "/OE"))
 (via (at 173.87333 44.6218) (size 0.6) (drill 0.3) (layers "F.Cu" "B.Cu") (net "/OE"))
 (via (at 167.884035 38.353635) (size 0.6) (drill 0.3) (layers "F.Cu" "B.Cu") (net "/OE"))
 (via (at 166.79483 35.5442) (size 0.6) (drill 0.3) (layers "F.Cu" "B.Cu") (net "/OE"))
 (segment (start 167.884035 38.632505) (end 167.884035 38.353635) (width 0.2) (layer "B.Cu") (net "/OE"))
 (segment (start 173.87333 44.6218) (end 167.884035 38.632505) (width 0.2) (layer "B.Cu") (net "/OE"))
 (segment (start 164.9984 35.3822) (end 166.63283 35.3822) (width 0.2) (layer "B.Cu") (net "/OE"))
 (segment (start 166.63283 35.3822) (end 166.79483 35.5442) (width 0.2) (layer "B.Cu") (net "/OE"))
 (segment (start 165.69483 36.35257) (end 165.69483 33.6588) (width 0.2) (layer "F.Cu") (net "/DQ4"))
 (segment (start 163.576 38.4714) (end 165.69483 36.35257) (width 0.2) (layer "F.Cu") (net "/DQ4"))
 (via (at 163.576 38.4714) (size 0.6) (drill 0.3) (layers "F.Cu" "B.Cu") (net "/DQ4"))
 (segment (start 163.2204 46.8062) (end 163.2204 38.827) (width 0.2) (layer "B.Cu") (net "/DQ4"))
 (segment (start 163.2204 38.827) (end 163.576 38.4714) (width 0.2) (layer "B.Cu") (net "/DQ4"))
 (segment (start 151.8666 58.16) (end 163.2204 46.8062) (width 0.2) (layer "B.Cu") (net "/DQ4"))
 (segment (start 166.19483 36.95437) (end 163.8808 39.2684) (width 0.2) (layer "F.Cu") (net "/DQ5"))
 (segment (start 166.19483 33.6588) (end 166.19483 36.95437) (width 0.2) (layer "F.Cu") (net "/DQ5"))
 (via (at 163.8808 39.2684) (size 0.6) (drill 0.3) (layers "F.Cu" "B.Cu") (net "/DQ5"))
 (segment (start 163.8808 39.2684) (end 163.8808 48.6858) (width 0.2) (layer "B.Cu") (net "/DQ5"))
 (segment (start 163.8808 48.6858) (end 151.8666 60.7) (width 0.2) (layer "B.Cu") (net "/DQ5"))
 (segment (start 167.5257 35.0901) (end 167.19483 34.75923) (width 0.2) (layer "F.Cu") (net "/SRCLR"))
 (segment (start 167.19483 34.75923) (end 167.19483 33.6588) (width 0.2) (layer "F.Cu") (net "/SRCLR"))
 (via (at 167.5257 35.0901) (size 0.6) (drill 0.3) (layers "F.Cu" "B.Cu") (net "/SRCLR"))
 (segment (start 171.5672 35.5442) (end 184.023 48) (width 0.2) (layer "B.Cu") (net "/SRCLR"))
 (segment (start 167.5257 35.0901) (end 167.9798 35.5442) (width 0.2) (layer "B.Cu") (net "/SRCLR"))
 (segment (start 167.9798 35.5442) (end 171.5672 35.5442) (width 0.2) (layer "B.Cu") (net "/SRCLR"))
 (segment (start 168.69483 38.39137) (end 168.69483 33.6588) (width 0.2) (layer "F.Cu") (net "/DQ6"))
 (segment (start 165.9128 39.0144) (end 168.0718 39.0144) (width 0.2) (layer "F.Cu") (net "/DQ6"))
 (segment (start 168.0718 39.0144) (end 168.69483 38.39137) (width 0.2) (layer "F.Cu") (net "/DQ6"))
 (via (at 165.9128 39.0144) (size 0.6) (drill 0.3) (layers "F.Cu" "B.Cu") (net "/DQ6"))
 (segment (start 165.9128 39.0144) (end 164.9984 39.9288) (width 0.2) (layer "B.Cu") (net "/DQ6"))
 (segment (start 164.9984 39.9288) (end 164.9984 50.1082) (width 0.2) (layer "B.Cu") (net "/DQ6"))
 (segment (start 164.9984 50.1082) (end 151.8666 63.24) (width 0.2) (layer "B.Cu") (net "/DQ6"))
 (segment (start 169.19483 35.9238) (end 173.39483 40.1238) (width 0.2) (layer "F.Cu") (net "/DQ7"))
 (segment (start 169.19483 33.6588) (end 169.19483 35.9238) (width 0.2) (layer "F.Cu") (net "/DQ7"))
 (segment (start 173.39483 44.25177) (end 151.8666 65.78) (width 0.2) (layer "F.Cu") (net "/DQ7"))
 (segment (start 173.39483 40.1238) (end 173.39483 44.25177) (width 0.2) (layer "F.Cu") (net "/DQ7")))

